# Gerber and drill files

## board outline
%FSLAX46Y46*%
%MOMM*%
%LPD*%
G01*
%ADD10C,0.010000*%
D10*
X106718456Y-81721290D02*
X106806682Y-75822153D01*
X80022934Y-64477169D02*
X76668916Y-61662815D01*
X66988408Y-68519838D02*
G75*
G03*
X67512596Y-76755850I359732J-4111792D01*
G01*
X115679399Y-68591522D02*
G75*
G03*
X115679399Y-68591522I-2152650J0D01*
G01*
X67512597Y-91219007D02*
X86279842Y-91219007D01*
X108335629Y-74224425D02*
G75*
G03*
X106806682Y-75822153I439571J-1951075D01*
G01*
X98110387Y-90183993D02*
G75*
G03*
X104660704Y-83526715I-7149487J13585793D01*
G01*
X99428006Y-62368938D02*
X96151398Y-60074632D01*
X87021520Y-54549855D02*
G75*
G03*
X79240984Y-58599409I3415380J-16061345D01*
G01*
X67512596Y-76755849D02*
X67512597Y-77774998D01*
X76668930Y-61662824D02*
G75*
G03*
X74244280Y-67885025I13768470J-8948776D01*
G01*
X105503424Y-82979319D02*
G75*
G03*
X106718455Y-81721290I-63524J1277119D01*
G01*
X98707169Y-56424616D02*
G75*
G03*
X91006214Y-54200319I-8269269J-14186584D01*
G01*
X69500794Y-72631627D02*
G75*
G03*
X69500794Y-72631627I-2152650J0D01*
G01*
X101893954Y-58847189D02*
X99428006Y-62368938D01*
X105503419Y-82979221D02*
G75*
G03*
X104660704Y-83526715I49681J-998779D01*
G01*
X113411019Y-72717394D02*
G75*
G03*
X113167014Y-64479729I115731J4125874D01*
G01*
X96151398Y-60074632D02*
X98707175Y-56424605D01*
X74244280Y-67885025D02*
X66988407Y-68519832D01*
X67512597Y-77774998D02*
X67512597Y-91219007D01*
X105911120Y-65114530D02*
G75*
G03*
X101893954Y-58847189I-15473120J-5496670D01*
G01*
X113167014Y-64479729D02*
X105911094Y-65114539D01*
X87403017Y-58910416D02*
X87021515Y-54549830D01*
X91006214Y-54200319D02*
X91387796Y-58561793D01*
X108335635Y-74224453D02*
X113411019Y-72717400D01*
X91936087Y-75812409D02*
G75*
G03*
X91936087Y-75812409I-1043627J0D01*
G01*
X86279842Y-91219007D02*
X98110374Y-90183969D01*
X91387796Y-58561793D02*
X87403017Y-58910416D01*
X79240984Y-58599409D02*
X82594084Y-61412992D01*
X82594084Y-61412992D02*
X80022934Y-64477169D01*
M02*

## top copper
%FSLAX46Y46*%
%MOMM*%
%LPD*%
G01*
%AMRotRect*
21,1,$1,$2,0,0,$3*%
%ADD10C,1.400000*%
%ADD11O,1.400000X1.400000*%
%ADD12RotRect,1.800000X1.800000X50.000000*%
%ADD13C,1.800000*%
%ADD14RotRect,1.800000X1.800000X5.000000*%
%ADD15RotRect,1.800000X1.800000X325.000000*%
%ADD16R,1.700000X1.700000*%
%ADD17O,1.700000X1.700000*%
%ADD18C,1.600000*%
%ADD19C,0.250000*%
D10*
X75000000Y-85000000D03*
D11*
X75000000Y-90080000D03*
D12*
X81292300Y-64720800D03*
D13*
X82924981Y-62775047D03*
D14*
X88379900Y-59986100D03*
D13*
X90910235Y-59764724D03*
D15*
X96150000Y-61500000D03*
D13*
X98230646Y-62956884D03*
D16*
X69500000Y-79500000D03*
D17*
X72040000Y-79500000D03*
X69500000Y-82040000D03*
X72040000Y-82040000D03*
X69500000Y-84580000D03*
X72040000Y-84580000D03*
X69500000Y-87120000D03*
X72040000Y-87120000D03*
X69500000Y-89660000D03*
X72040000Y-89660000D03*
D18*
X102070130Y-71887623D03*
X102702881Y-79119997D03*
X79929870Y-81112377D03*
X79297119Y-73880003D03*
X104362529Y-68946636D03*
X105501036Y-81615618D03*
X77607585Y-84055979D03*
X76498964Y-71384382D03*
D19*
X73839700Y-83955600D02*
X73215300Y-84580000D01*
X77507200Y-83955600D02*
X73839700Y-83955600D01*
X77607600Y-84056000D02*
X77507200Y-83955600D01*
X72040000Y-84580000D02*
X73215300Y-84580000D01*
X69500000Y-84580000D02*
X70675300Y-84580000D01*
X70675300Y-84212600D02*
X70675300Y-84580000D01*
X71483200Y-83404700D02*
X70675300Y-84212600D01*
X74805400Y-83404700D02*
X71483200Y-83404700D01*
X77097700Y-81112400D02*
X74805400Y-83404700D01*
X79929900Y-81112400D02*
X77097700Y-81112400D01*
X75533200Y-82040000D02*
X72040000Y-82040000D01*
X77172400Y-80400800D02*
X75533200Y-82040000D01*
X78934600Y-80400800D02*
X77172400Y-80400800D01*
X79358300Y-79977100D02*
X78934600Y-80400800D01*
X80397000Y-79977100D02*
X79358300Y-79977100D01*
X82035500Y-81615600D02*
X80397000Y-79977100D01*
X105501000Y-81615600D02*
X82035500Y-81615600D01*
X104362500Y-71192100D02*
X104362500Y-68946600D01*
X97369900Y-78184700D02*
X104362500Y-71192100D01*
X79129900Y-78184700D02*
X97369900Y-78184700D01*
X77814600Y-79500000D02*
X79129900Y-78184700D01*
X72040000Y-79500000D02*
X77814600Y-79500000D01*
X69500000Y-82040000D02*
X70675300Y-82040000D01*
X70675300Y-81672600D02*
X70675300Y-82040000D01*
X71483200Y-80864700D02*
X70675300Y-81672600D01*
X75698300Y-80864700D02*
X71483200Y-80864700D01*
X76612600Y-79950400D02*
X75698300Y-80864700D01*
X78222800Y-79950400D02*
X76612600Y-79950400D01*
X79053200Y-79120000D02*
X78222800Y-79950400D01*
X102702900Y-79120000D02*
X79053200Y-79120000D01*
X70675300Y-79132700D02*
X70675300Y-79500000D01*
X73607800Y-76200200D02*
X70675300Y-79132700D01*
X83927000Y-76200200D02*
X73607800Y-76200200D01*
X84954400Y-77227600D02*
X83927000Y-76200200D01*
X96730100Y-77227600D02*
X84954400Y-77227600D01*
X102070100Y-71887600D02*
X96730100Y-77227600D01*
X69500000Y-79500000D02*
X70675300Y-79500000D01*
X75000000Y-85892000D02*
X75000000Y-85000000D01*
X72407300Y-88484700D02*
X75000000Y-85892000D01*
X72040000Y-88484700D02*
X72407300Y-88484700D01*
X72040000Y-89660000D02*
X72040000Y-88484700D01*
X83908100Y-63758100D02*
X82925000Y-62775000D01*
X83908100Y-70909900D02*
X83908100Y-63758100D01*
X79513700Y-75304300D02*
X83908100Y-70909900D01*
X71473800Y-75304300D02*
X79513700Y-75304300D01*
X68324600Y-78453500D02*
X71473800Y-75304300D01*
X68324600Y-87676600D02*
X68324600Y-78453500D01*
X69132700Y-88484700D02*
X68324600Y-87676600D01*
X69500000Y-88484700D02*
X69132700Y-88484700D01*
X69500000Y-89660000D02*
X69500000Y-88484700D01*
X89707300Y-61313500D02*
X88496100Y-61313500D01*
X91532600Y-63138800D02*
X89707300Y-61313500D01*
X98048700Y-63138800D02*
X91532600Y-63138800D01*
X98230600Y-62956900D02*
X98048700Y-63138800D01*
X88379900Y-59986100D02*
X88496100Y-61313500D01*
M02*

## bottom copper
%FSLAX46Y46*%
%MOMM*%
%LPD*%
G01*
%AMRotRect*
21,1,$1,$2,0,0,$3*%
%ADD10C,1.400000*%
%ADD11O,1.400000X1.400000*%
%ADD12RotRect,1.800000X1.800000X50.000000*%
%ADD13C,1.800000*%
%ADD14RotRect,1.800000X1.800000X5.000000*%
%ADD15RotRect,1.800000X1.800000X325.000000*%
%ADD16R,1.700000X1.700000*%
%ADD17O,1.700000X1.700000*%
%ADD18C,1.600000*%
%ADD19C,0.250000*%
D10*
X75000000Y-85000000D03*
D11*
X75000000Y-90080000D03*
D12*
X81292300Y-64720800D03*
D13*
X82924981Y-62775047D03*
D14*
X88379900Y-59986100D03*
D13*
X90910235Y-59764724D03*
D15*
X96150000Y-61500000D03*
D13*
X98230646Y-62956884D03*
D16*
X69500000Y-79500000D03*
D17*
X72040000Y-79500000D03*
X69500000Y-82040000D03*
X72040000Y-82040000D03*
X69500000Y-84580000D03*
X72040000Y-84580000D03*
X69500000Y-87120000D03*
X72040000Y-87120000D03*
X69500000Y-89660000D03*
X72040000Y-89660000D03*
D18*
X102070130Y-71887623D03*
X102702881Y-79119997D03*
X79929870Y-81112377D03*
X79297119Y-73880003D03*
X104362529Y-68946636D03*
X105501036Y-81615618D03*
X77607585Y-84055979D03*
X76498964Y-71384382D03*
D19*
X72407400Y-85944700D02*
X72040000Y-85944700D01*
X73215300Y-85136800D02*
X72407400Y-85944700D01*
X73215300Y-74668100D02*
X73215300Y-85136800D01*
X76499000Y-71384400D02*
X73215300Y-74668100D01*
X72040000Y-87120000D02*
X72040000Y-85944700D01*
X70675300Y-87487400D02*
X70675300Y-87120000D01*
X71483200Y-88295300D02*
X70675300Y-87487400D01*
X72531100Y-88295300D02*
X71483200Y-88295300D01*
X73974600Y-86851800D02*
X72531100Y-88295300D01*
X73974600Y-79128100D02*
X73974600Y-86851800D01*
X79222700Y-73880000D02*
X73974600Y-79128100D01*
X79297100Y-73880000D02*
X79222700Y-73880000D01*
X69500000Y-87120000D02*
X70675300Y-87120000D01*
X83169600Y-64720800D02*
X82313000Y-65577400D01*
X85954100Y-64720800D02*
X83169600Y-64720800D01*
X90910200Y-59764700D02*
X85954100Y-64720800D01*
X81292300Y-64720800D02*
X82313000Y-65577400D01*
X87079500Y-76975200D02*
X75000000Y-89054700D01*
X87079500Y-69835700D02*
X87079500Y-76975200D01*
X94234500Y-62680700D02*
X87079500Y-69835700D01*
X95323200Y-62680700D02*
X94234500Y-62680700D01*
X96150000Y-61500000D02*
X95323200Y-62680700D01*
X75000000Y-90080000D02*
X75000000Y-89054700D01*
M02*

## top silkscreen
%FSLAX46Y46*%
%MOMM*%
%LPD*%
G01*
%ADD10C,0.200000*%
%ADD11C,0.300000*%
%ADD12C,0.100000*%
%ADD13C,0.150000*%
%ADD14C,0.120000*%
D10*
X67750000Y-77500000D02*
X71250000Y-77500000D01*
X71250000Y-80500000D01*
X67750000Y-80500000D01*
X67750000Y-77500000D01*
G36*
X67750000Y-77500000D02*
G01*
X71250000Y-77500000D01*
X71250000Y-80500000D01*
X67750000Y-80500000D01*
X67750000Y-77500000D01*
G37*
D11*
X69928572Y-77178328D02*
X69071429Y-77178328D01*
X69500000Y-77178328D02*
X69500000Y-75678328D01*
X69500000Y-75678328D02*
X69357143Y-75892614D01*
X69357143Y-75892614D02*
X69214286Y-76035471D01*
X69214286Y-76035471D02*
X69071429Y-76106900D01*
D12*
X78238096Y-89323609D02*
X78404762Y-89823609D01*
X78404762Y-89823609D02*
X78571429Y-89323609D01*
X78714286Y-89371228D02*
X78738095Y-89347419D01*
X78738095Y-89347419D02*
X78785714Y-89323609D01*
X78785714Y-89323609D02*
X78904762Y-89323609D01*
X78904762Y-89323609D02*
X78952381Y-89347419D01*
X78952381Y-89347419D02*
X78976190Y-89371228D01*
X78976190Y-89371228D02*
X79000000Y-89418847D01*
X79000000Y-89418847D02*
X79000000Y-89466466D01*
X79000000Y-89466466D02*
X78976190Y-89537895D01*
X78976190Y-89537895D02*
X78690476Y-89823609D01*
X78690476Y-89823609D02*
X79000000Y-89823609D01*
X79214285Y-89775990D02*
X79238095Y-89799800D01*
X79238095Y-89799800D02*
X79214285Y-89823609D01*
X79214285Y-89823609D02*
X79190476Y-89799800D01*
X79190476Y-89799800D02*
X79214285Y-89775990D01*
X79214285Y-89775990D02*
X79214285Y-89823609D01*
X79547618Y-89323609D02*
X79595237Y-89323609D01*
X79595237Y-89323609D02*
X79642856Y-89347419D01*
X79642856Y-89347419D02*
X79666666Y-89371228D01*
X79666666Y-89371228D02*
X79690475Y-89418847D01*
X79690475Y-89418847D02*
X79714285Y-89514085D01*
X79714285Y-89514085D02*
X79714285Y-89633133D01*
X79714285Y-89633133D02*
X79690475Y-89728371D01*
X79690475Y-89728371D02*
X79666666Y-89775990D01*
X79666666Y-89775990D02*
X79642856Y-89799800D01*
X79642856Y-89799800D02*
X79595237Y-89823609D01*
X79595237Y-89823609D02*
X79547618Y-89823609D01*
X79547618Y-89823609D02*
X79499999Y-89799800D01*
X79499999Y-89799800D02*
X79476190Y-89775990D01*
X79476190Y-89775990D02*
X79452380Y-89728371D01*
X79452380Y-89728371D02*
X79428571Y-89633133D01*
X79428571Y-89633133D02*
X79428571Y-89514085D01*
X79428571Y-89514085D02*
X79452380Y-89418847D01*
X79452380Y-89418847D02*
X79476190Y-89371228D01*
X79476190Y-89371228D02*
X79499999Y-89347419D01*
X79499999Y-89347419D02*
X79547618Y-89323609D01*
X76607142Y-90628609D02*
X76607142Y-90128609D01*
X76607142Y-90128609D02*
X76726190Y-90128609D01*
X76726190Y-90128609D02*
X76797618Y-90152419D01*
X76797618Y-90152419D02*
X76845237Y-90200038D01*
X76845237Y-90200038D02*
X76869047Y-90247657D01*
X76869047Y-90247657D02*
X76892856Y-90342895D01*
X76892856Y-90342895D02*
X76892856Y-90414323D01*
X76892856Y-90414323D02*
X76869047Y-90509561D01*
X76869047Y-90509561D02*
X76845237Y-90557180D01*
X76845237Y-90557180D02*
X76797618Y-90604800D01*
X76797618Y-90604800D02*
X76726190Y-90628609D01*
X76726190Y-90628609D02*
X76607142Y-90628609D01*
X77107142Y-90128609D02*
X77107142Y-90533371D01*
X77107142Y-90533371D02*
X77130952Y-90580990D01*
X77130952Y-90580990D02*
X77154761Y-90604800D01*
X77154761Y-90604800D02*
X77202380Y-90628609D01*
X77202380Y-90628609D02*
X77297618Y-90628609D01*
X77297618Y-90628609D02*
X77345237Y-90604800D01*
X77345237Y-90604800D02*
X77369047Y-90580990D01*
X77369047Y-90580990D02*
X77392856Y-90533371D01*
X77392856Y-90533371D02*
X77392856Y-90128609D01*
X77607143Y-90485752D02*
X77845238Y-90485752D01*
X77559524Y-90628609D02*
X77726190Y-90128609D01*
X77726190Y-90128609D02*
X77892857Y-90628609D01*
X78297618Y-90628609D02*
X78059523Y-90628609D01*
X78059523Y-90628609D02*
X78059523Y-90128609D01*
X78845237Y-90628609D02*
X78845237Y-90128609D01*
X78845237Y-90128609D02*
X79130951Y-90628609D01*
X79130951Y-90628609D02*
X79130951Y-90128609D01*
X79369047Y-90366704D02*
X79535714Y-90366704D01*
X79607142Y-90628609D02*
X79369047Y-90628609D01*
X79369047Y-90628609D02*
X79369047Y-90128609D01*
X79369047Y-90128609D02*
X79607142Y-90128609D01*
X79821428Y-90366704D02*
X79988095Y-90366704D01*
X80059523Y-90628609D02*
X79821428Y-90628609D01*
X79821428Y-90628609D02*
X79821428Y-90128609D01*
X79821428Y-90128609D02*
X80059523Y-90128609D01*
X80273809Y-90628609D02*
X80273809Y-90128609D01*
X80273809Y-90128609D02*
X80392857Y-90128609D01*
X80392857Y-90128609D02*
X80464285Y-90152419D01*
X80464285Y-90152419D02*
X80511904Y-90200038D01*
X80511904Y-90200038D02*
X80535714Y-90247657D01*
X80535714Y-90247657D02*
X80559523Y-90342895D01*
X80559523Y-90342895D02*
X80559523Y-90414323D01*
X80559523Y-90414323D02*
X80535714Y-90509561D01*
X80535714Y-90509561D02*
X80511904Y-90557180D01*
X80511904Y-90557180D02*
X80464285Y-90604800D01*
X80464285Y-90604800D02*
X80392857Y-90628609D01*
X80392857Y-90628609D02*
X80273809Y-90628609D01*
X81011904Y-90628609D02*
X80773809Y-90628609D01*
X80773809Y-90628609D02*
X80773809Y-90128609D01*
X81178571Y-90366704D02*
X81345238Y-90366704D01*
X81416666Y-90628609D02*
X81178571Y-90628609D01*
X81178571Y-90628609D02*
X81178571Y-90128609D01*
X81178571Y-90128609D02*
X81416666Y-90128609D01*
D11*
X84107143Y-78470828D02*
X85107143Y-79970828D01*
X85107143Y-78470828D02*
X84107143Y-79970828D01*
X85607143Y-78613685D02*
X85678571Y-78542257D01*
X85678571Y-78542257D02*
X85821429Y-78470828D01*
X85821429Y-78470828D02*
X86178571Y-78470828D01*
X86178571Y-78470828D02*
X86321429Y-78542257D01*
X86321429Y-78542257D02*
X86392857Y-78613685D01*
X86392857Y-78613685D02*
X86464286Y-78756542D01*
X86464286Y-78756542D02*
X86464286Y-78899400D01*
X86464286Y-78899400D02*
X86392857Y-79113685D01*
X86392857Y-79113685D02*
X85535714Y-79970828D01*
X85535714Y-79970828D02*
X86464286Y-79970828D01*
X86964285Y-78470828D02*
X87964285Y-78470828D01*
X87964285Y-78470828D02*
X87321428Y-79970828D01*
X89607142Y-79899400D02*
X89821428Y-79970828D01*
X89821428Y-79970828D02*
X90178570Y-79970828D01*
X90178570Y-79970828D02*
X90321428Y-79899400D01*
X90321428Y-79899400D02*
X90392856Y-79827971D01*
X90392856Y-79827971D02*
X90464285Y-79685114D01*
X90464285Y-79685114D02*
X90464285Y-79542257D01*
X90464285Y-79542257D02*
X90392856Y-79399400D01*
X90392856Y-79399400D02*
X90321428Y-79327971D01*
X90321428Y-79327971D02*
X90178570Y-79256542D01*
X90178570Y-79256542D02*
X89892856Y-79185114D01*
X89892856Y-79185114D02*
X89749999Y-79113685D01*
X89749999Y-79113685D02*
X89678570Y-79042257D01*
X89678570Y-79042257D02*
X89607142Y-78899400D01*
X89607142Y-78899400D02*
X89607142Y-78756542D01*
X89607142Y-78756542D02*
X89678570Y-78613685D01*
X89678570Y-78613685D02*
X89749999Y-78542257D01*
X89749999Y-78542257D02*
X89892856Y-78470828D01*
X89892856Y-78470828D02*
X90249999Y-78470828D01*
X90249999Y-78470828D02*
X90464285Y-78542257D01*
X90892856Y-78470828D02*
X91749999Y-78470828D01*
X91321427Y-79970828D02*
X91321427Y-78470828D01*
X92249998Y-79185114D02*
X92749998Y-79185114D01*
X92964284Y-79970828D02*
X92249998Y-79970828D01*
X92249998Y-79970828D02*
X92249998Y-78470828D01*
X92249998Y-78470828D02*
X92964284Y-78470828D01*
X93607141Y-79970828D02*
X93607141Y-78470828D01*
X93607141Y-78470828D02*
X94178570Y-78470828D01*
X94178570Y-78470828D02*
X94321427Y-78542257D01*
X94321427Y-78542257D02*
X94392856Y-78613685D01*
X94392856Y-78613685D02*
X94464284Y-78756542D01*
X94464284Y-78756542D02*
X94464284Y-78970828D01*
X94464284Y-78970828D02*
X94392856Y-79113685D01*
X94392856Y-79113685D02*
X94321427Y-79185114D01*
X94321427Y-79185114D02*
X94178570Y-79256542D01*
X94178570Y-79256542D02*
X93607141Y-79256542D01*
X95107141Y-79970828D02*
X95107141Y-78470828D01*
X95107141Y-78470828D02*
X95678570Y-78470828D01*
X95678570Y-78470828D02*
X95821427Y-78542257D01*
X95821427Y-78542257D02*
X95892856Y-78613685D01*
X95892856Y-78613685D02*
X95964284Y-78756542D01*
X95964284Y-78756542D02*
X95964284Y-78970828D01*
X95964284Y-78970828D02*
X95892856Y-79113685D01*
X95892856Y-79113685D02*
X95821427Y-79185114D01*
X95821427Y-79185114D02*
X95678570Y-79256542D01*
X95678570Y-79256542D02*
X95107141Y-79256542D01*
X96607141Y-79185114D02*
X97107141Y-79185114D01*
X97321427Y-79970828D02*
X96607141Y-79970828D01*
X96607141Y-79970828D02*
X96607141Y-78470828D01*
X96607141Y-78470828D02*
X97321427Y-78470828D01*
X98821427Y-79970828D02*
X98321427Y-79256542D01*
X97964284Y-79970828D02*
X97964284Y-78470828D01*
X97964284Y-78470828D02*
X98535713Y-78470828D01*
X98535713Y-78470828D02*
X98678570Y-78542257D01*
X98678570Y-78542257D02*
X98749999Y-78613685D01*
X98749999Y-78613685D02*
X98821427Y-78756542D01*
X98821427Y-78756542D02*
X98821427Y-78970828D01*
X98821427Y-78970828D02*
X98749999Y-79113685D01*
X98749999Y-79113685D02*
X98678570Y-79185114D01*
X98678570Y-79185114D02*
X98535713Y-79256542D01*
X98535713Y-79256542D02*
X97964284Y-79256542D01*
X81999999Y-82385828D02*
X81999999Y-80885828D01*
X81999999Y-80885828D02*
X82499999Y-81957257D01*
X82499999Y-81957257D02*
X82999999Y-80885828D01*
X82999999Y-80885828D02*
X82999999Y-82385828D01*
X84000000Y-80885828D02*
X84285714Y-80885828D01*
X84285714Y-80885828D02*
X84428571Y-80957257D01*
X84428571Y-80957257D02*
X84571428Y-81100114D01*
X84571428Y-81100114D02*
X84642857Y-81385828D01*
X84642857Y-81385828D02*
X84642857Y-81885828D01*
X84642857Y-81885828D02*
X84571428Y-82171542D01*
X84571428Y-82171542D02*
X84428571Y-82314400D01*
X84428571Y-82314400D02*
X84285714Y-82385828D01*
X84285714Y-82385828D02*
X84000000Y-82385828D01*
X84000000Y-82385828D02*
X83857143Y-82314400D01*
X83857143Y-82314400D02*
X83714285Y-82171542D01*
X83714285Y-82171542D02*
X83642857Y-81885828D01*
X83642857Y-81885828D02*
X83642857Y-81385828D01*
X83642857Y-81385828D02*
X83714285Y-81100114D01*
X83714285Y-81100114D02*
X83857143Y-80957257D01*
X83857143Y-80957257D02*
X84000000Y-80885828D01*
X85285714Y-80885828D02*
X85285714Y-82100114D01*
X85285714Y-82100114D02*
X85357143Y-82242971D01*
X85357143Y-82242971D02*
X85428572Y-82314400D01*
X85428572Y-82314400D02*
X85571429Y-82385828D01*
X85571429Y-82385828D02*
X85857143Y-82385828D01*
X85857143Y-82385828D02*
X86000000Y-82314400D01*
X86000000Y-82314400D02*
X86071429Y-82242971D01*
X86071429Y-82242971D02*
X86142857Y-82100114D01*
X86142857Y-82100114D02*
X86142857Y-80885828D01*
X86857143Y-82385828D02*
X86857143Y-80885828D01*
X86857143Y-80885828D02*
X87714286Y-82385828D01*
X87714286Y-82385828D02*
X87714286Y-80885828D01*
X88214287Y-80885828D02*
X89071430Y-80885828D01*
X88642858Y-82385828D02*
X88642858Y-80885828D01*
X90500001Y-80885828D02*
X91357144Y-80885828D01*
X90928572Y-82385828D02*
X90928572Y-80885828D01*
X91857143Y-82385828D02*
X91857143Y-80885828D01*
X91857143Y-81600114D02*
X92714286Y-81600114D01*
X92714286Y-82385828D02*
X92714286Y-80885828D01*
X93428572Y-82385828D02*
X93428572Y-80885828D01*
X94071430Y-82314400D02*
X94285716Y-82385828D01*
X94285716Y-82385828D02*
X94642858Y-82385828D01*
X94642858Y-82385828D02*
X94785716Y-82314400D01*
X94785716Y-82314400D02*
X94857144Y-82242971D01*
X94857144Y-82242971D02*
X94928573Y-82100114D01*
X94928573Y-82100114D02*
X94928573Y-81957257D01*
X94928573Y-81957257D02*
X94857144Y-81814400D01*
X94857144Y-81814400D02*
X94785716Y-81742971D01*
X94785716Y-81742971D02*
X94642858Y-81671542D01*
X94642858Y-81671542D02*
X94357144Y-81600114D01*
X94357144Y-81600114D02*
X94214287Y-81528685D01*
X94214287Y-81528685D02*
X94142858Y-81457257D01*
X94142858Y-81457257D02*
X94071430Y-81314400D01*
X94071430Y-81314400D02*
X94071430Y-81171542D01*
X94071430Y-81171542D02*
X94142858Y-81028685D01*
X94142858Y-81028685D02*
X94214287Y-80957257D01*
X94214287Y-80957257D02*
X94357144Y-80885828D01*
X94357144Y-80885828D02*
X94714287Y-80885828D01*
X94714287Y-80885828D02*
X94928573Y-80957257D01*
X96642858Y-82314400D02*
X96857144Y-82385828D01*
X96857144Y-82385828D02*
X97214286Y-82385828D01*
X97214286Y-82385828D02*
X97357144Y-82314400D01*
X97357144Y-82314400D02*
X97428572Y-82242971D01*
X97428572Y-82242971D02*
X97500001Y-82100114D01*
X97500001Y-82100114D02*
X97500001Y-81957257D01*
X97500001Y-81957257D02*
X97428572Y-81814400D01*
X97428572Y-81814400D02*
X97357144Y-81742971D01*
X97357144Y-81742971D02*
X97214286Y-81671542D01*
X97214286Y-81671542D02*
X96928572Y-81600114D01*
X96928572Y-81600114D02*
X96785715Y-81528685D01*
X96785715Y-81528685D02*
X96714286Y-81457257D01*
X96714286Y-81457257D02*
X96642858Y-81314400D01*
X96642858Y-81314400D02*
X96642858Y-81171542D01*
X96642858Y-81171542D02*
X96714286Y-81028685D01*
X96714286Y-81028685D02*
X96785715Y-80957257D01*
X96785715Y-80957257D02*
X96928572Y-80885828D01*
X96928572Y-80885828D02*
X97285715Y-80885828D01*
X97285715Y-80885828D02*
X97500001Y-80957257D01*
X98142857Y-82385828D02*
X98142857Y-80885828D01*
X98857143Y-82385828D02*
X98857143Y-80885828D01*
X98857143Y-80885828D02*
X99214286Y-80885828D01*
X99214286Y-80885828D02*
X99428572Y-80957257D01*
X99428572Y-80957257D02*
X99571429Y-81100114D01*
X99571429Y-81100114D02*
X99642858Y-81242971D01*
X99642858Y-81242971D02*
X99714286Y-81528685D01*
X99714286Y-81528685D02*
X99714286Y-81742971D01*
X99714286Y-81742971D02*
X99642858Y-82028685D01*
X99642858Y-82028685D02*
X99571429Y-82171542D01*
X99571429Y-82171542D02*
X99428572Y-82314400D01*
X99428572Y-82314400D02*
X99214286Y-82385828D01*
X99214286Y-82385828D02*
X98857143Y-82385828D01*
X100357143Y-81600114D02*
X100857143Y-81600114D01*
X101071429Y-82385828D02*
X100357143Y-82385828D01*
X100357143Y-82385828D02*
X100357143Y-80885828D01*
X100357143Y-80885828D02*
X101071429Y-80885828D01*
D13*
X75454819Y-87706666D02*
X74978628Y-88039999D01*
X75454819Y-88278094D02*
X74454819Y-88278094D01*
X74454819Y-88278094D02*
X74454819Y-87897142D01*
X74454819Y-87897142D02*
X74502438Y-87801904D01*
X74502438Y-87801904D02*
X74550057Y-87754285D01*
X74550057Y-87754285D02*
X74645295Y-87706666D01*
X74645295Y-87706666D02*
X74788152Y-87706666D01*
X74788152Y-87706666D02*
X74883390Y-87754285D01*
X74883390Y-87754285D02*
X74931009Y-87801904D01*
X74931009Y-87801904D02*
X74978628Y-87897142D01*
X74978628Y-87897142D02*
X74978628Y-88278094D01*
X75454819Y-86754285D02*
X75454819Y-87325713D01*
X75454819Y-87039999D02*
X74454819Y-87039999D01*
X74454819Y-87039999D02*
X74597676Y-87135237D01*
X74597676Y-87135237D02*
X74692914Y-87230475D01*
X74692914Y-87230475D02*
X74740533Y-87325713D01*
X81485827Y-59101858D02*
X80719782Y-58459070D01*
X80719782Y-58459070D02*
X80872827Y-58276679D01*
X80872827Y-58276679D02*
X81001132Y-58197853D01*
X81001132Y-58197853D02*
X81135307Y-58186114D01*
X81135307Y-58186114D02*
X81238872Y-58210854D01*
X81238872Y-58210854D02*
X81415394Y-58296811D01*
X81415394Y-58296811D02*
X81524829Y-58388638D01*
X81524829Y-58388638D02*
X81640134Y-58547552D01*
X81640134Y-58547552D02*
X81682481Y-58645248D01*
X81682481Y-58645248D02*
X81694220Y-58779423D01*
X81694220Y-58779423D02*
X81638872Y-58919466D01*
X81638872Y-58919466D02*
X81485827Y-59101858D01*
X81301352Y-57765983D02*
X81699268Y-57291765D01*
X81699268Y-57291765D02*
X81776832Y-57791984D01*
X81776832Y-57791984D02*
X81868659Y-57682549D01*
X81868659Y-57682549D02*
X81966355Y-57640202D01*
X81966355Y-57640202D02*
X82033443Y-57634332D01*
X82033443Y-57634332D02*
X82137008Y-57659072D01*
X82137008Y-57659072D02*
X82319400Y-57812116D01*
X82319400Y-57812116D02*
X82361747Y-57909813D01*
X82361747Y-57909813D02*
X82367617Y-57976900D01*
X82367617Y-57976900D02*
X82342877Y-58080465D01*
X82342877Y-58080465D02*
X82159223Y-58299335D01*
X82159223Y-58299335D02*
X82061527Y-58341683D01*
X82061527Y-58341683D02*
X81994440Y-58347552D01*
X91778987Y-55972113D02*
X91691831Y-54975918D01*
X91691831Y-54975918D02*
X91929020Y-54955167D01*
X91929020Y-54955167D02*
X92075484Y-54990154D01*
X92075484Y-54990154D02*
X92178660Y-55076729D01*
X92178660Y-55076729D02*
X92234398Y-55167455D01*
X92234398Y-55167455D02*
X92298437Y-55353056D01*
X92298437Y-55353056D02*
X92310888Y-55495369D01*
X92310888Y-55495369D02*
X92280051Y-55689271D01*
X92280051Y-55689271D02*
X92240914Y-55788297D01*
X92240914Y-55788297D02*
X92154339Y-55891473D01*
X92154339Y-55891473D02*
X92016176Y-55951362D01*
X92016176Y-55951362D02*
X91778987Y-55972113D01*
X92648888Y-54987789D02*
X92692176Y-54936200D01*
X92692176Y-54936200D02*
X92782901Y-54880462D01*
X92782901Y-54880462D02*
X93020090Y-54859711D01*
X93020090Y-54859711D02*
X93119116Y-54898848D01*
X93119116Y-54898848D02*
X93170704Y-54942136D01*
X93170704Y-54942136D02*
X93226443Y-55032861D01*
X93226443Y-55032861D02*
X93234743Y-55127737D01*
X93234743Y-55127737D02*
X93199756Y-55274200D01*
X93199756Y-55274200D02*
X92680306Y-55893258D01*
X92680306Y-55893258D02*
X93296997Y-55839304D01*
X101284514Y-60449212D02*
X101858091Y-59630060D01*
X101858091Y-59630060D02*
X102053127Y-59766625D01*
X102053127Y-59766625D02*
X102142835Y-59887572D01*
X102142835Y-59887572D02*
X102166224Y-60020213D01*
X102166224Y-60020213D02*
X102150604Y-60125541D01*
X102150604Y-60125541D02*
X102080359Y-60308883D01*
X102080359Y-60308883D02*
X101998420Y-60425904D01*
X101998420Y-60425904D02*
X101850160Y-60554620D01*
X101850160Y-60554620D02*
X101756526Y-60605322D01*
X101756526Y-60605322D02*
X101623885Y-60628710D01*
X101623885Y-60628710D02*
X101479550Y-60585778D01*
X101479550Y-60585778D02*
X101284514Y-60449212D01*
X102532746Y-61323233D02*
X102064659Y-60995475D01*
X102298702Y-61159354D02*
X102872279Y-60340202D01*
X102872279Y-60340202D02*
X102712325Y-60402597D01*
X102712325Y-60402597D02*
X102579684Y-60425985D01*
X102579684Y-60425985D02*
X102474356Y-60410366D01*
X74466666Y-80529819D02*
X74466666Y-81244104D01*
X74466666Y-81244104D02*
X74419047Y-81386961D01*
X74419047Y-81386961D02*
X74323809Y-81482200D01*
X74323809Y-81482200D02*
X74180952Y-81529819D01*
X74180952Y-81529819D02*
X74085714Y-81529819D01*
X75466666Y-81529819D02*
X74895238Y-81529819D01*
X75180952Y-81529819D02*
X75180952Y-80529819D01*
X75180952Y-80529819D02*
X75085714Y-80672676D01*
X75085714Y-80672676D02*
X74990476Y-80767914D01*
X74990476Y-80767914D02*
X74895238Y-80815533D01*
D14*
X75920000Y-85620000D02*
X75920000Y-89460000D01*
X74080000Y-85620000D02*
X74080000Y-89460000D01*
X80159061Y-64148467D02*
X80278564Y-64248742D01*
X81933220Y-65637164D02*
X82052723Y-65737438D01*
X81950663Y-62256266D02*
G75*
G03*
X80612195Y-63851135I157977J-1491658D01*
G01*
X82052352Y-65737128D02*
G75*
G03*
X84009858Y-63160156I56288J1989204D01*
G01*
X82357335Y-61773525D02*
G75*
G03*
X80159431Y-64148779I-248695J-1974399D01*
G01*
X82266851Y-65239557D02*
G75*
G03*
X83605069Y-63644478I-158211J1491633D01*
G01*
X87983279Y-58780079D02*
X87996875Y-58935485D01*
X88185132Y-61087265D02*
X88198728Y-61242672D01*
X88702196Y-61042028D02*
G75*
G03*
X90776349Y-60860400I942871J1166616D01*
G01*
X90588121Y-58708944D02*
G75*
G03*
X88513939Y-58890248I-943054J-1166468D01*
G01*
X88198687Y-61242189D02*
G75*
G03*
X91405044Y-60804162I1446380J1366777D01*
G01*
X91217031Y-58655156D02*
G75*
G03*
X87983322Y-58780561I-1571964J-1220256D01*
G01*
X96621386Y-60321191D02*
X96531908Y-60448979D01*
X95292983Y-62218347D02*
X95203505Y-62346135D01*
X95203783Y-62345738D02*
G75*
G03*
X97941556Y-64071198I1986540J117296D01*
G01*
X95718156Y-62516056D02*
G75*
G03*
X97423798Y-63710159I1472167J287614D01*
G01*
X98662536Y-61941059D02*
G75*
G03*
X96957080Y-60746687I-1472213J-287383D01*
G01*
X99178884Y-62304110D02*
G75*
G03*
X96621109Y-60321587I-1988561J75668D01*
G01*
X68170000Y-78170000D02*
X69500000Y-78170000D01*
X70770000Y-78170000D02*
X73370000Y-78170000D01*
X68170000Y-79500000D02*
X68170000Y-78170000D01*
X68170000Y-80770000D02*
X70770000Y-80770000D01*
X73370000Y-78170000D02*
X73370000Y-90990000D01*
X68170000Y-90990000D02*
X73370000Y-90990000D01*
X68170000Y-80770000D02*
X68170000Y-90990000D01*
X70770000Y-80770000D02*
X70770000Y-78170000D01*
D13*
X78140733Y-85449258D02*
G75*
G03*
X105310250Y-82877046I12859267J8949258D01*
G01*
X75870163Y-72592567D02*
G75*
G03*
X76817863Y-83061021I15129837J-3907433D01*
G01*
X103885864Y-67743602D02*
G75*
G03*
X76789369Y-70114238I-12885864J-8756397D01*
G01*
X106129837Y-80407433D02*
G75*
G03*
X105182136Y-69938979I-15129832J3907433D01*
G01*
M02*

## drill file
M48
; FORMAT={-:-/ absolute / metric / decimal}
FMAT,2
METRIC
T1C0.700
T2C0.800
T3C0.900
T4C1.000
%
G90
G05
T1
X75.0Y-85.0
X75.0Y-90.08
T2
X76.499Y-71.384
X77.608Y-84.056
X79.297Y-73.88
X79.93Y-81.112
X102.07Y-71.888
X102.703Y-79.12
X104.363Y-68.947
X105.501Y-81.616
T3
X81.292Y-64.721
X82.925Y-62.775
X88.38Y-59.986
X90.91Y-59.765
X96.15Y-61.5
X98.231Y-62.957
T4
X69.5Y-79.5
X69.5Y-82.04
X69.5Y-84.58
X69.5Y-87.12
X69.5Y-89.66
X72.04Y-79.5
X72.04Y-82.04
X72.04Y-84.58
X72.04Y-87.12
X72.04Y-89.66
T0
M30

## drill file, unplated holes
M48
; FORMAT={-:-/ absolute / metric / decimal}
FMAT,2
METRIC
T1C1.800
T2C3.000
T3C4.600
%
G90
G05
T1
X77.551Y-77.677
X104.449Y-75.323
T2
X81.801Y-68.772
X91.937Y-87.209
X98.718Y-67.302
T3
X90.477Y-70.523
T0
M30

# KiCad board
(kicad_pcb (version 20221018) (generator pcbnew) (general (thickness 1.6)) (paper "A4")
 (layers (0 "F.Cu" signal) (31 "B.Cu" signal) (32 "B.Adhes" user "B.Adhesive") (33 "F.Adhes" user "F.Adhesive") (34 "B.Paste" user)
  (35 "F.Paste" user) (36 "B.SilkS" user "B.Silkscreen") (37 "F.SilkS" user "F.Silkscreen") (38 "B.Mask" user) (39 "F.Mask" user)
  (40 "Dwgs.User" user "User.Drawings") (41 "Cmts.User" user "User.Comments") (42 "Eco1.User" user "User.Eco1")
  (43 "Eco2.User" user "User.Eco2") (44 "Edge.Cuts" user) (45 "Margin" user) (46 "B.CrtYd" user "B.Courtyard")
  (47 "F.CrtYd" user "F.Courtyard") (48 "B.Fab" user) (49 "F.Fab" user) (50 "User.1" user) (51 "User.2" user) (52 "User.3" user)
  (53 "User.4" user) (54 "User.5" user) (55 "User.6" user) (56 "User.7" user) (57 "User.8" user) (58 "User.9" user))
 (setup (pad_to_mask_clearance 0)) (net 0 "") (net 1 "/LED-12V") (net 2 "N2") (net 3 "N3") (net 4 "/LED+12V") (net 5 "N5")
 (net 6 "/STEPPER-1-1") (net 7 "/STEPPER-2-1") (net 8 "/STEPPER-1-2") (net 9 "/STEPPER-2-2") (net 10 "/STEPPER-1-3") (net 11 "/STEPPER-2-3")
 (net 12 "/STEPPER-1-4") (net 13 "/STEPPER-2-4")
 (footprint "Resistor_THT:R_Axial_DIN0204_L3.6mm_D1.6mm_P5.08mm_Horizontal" (layer "F.Cu") (at 75 85 -90)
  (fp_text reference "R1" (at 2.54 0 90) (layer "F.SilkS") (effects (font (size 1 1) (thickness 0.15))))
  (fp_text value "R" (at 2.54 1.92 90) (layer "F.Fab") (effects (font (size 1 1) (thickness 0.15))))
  (fp_line (start 0.62 -0.92) (end 4.46 -0.92) (stroke (width 0.12) (type solid)) (layer "F.SilkS"))
  (fp_line (start 0.62 0.92) (end 4.46 0.92) (stroke (width 0.12) (type solid)) (layer "F.SilkS"))
  (pad "1" thru_hole circle (at 0 0 270) (size 1.4 1.4) (drill 0.7) (layers "*.Cu" "*.Mask") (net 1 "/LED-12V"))
  (pad "2" thru_hole oval (at 5.08 0 270) (size 1.4 1.4) (drill 0.7) (layers "*.Cu" "*.Mask") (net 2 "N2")))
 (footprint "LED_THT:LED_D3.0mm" (layer "F.Cu") (at 81.2923 64.7208 50)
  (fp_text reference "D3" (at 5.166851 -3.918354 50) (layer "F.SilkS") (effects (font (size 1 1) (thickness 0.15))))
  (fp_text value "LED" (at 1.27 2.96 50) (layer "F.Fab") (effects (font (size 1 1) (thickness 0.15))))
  (fp_line (start -0.29 -1.236) (end -0.29 -1.08) (stroke (width 0.12) (type solid)) (layer "F.SilkS"))
  (fp_line (start -0.29 1.08) (end -0.29 1.236) (stroke (width 0.12) (type solid)) (layer "F.SilkS"))
  (fp_arc (start -0.29 -1.235516) (mid 1.366488 -1.987659) (end 2.942335 -1.078608) (stroke (width 0.12) (type solid)) (layer "F.SilkS"))
  (fp_arc (start 0.229039 -1.08) (mid 1.270117 -1.5) (end 2.31113 -1.079837) (stroke (width 0.12) (type solid)) (layer "F.SilkS"))
  (fp_arc (start 2.31113 1.079837) (mid 1.270117 1.5) (end 0.229039 1.08) (stroke (width 0.12) (type solid)) (layer "F.SilkS"))
  (fp_arc (start 2.942335 1.078608) (mid 1.366487 1.987659) (end -0.29 1.235516) (stroke (width 0.12) (type solid)) (layer "F.SilkS"))
  (pad "1" thru_hole rect (at 0 0 50) (size 1.8 1.8) (drill 0.9) (layers "*.Cu" "*.Mask") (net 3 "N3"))
  (pad "2" thru_hole circle (at 2.54 0 50) (size 1.8 1.8) (drill 0.9) (layers "*.Cu" "*.Mask") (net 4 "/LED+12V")))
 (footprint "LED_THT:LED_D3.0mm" (layer "F.Cu") (at 88.3799 59.9861 5)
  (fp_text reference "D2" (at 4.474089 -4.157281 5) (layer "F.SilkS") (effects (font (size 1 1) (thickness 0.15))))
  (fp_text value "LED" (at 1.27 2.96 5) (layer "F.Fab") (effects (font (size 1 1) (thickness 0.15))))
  (fp_line (start -0.29 -1.236) (end -0.29 -1.08) (stroke (width 0.12) (type solid)) (layer "F.SilkS"))
  (fp_line (start -0.29 1.08) (end -0.29 1.236) (stroke (width 0.12) (type solid)) (layer "F.SilkS"))
  (fp_arc (start -0.29 -1.235516) (mid 1.366488 -1.987659) (end 2.942335 -1.078608) (stroke (width 0.12) (type solid)) (layer "F.SilkS"))
  (fp_arc (start 0.229039 -1.08) (mid 1.270118 -1.5) (end 2.31113 -1.079837) (stroke (width 0.12) (type solid)) (layer "F.SilkS"))
  (fp_arc (start 2.31113 1.079837) (mid 1.270118 1.5) (end 0.229039 1.08) (stroke (width 0.12) (type solid)) (layer "F.SilkS"))
  (fp_arc (start 2.942335 1.078608) (mid 1.366488 1.987659) (end -0.29 1.235516) (stroke (width 0.12) (type solid)) (layer "F.SilkS"))
  (pad "1" thru_hole rect (at 0 0 5) (size 1.8 1.8) (drill 0.9) (layers "*.Cu" "*.Mask") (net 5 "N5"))
  (pad "2" thru_hole circle (at 2.54 0 5) (size 1.8 1.8) (drill 0.9) (layers "*.Cu" "*.Mask") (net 3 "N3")))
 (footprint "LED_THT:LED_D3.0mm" (layer "F.Cu") (at 96.15 61.5 -35)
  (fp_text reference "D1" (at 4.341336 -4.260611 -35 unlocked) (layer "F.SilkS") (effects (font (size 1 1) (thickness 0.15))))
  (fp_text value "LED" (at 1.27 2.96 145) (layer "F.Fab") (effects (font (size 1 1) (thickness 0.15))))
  (fp_line (start -0.29 -1.236) (end -0.29 -1.08) (stroke (width 0.12) (type solid)) (layer "F.SilkS"))
  (fp_line (start -0.29 1.08) (end -0.29 1.236) (stroke (width 0.12) (type solid)) (layer "F.SilkS"))
  (fp_arc (start -0.29 -1.235516) (mid 1.366487 -1.987659) (end 2.942335 -1.078608) (stroke (width 0.12) (type solid)) (layer "F.SilkS"))
  (fp_arc (start 0.229039 -1.08) (mid 1.270118 -1.5) (end 2.31113 -1.079837) (stroke (width 0.12) (type solid)) (layer "F.SilkS"))
  (fp_arc (start 2.31113 1.079837) (mid 1.270117 1.5) (end 0.229039 1.08) (stroke (width 0.12) (type solid)) (layer "F.SilkS"))
  (fp_arc (start 2.942335 1.078608) (mid 1.366487 1.987659) (end -0.29 1.235516) (stroke (width 0.12) (type solid)) (layer "F.SilkS"))
  (pad "1" thru_hole rect (at 0 0 325) (size 1.8 1.8) (drill 0.9) (layers "*.Cu" "*.Mask") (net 2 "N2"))
  (pad "2" thru_hole circle (at 2.54 0 325) (size 1.8 1.8) (drill 0.9) (layers "*.Cu" "*.Mask") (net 5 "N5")))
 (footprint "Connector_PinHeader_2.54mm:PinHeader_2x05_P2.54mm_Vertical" (layer "F.Cu") (at 69.5 79.5)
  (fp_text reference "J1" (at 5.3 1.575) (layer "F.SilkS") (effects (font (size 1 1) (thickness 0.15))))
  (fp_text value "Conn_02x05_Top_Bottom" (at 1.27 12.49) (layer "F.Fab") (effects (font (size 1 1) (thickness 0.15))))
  (fp_line (start -1.33 -1.33) (end 0 -1.33) (stroke (width 0.12) (type solid)) (layer "F.SilkS"))
  (fp_line (start -1.33 0) (end -1.33 -1.33) (stroke (width 0.12) (type solid)) (layer "F.SilkS"))
  (fp_line (start -1.33 1.27) (end -1.33 11.49) (stroke (width 0.12) (type solid)) (layer "F.SilkS"))
  (fp_line (start -1.33 1.27) (end 1.27 1.27) (stroke (width 0.12) (type solid)) (layer "F.SilkS"))
  (fp_line (start -1.33 11.49) (end 3.87 11.49) (stroke (width 0.12) (type solid)) (layer "F.SilkS"))
  (fp_line (start 1.27 -1.33) (end 3.87 -1.33) (stroke (width 0.12) (type solid)) (layer "F.SilkS"))
  (fp_line (start 1.27 1.27) (end 1.27 -1.33) (stroke (width 0.12) (type solid)) (layer "F.SilkS"))
  (fp_line (start 3.87 -1.33) (end 3.87 11.49) (stroke (width 0.12) (type solid)) (layer "F.SilkS"))
  (pad "1" thru_hole rect (at 0 0) (size 1.7 1.7) (drill 1) (layers "*.Cu" "*.Mask") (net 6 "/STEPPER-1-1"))
  (pad "2" thru_hole oval (at 2.54 0) (size 1.7 1.7) (drill 1) (layers "*.Cu" "*.Mask") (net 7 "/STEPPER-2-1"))
  (pad "3" thru_hole oval (at 0 2.54) (size 1.7 1.7) (drill 1) (layers "*.Cu" "*.Mask") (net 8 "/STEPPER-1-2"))
  (pad "4" thru_hole oval (at 2.54 2.54) (size 1.7 1.7) (drill 1) (layers "*.Cu" "*.Mask") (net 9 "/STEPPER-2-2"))
  (pad "5" thru_hole oval (at 0 5.08) (size 1.7 1.7) (drill 1) (layers "*.Cu" "*.Mask") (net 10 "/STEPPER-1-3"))
  (pad "6" thru_hole oval (at 2.54 5.08) (size 1.7 1.7) (drill 1) (layers "*.Cu" "*.Mask") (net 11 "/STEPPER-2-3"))
  (pad "7" thru_hole oval (at 0 7.62) (size 1.7 1.7) (drill 1) (layers "*.Cu" "*.Mask") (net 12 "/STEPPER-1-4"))
  (pad "8" thru_hole oval (at 2.54 7.62) (size 1.7 1.7) (drill 1) (layers "*.Cu" "*.Mask") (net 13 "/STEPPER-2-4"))
  (pad "9" thru_hole oval (at 0 10.16) (size 1.7 1.7) (drill 1) (layers "*.Cu" "*.Mask") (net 4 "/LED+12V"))
  (pad "10" thru_hole oval (at 2.54 10.16) (size 1.7 1.7) (drill 1) (layers "*.Cu" "*.Mask") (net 1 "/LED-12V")))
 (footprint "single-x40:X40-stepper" (layer "B.Cu") (at 91 76.5 -175)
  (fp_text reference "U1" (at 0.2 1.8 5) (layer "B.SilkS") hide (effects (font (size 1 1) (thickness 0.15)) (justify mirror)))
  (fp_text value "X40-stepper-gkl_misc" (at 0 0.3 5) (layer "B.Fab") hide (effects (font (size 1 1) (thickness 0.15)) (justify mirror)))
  (fp_arc (start -14.7 5.3) (mid -15.626189 0.047138) (end -14.731708 -5.211216) (stroke (width 0.15) (type solid)) (layer "F.SilkS"))
  (fp_arc (start -13.7 -7.6) (mid -0.111624 -15.666446) (end 13.590314 -7.794445) (stroke (width 0.15) (type solid)) (layer "F.SilkS"))
  (fp_arc (start 13.6 7.6) (mid 0 15.579474) (end -13.6 7.6) (stroke (width 0.15) (type solid)) (layer "F.SilkS"))
  (fp_arc (start 14.7 -5.3) (mid 15.626189 -0.047138) (end 14.731708 5.211216) (stroke (width 0.15) (type solid)) (layer "F.SilkS"))
  (pad "" np_thru_hole circle (at -13.5 0 185) (size 1.8 1.8) (drill 1.8) (layers "*.Cu" "*.Mask"))
  (pad "" np_thru_hole circle (at -8.49 8.49 185) (size 3 3) (drill 3) (layers "*.Cu" "*.Mask"))
  (pad "" np_thru_hole circle (at 0 -10.75 185) (size 3 3) (drill 3) (layers "*.Cu" "*.Mask"))
  (pad "" np_thru_hole circle (at 0 6 185) (size 4.6 4.6) (drill 4.6) (layers "*.Cu" "*.Mask"))
  (pad "" np_thru_hole circle (at 8.49 8.5 185) (size 3 3) (drill 3) (layers "*.Cu" "*.Mask"))
  (pad "" np_thru_hole circle (at 13.5 0 185) (size 1.8 1.8) (drill 1.8) (layers "*.Cu" "*.Mask"))
  (pad "1" thru_hole circle (at -11.43 3.63 185) (size 1.6 1.6) (drill 0.8) (layers "*.Cu" "*.Mask") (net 6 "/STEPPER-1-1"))
  (pad "2" thru_hole circle (at -11.43 -3.63 185) (size 1.6 1.6) (drill 0.8) (layers "*.Cu" "*.Mask") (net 8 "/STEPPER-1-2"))
  (pad "3" thru_hole circle (at 11.43 -3.63 185) (size 1.6 1.6) (drill 0.8) (layers "*.Cu" "*.Mask") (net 10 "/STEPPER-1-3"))
  (pad "4" thru_hole circle (at 11.43 3.63 185) (size 1.6 1.6) (drill 0.8) (layers "*.Cu" "*.Mask") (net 12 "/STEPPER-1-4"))
  (pad "5" thru_hole circle (at -13.97 6.36 185) (size 1.6 1.6) (drill 0.8) (layers "*.Cu" "*.Mask") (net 7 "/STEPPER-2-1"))
  (pad "6" thru_hole circle (at -14 -6.36 185) (size 1.6 1.6) (drill 0.8) (layers "*.Cu" "*.Mask") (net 9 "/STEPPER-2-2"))
  (pad "7" thru_hole circle (at 14 -6.36 185) (size 1.6 1.6) (drill 0.8) (layers "*.Cu" "*.Mask") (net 11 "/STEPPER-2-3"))
  (pad "8" thru_hole circle (at 14 6.36 185) (size 1.6 1.6) (drill 0.8) (layers "*.Cu" "*.Mask") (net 13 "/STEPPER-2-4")))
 (gr_rect (start 67.75 77.5) (end 71.25 80.5) (stroke (width 0.2) (type solid)) (fill solid) (layer "F.SilkS"))
 (gr_line (start 106.718456 81.72129) (end 106.806682 75.822153) (stroke (width 0.01) (type solid)) (layer "Edge.Cuts"))
 (gr_line (start 80.022934 64.477169) (end 76.668916 61.662815) (stroke (width 0.01) (type solid)) (layer "Edge.Cuts"))
 (gr_arc (start 67.512596 76.755851) (mid 63.228977 72.893795) (end 66.988407 68.519832) (stroke (width 0.01) (type solid))
  (layer "Edge.Cuts"))
 (gr_circle (center 113.526749 68.591522) (end 115.679399 68.591522) (stroke (width 0.01) (type solid)) (fill none) (layer "Edge.Cuts"))
 (gr_line (start 67.512597 91.219007) (end 86.279842 91.219007) (stroke (width 0.01) (type solid)) (layer "Edge.Cuts"))
 (gr_arc (start 106.806682 75.822153) (mid 107.330253 74.792764) (end 108.335635 74.224453) (stroke (width 0.01) (type solid))
  (layer "Edge.Cuts"))
 (gr_arc (start 104.660704 83.526715) (mid 101.904066 87.365541) (end 98.110374 90.183969) (stroke (width 0.01) (type solid))
  (layer "Edge.Cuts"))
 (gr_line (start 99.428006 62.368938) (end 96.151398 60.074632) (stroke (width 0.01) (type solid)) (layer "Edge.Cuts"))
 (gr_arc (start 79.240984 58.599409) (mid 82.855853 56.045494) (end 87.021515 54.54983) (stroke (width 0.01) (type solid))
  (layer "Edge.Cuts"))
 (gr_line (start 67.512596 76.755849) (end 67.512597 77.774998) (stroke (width 0.01) (type solid)) (layer "Edge.Cuts"))
 (gr_arc (start 74.24428 67.885025) (mid 75.136963 64.649366) (end 76.668916 61.662815) (stroke (width 0.01) (type solid))
  (layer "Edge.Cuts"))
 (gr_arc (start 106.718456 81.72129) (mid 106.359644 82.590491) (end 105.503421 82.979257) (stroke (width 0.01) (type solid))
  (layer "Edge.Cuts"))
 (gr_arc (start 91.006214 54.200319) (mid 94.994501 54.835344) (end 98.707175 56.424605) (stroke (width 0.01) (type solid))
  (layer "Edge.Cuts"))
 (gr_circle (center 67.348144 72.631627) (end 69.500794 72.631627) (stroke (width 0.01) (type solid)) (fill none) (layer "Edge.Cuts"))
 (gr_line (start 101.893954 58.847189) (end 99.428006 62.368938) (stroke (width 0.01) (type solid)) (layer "Edge.Cuts"))
 (gr_arc (start 104.660704 83.526715) (mid 105.008299 83.13944) (end 105.503421 82.979257) (stroke (width 0.01) (type solid))
  (layer "Edge.Cuts"))
 (gr_arc (start 113.167014 64.479729) (mid 117.65244 68.469317) (end 113.411019 72.7174) (stroke (width 0.01) (type solid))
  (layer "Edge.Cuts"))
 (gr_line (start 96.151398 60.074632) (end 98.707175 56.424605) (stroke (width 0.01) (type solid)) (layer "Edge.Cuts"))
 (gr_line (start 74.24428 67.885025) (end 66.988407 68.519832) (stroke (width 0.01) (type solid)) (layer "Edge.Cuts"))
 (gr_line (start 67.512597 77.774998) (end 67.512597 91.219007) (stroke (width 0.01) (type solid)) (layer "Edge.Cuts"))
 (gr_arc (start 101.893954 58.847189) (mid 104.262373 61.750214) (end 105.911094 65.114539) (stroke (width 0.01) (type solid))
  (layer "Edge.Cuts"))
 (gr_line (start 113.167014 64.479729) (end 105.911094 65.114539) (stroke (width 0.01) (type solid)) (layer "Edge.Cuts"))
 (gr_line (start 87.403017 58.910416) (end 87.021515 54.54983) (stroke (width 0.01) (type solid)) (layer "Edge.Cuts"))
 (gr_line (start 91.006214 54.200319) (end 91.387796 58.561793) (stroke (width 0.01) (type solid)) (layer "Edge.Cuts"))
 (gr_line (start 108.335635 74.224453) (end 113.411019 72.7174) (stroke (width 0.01) (type solid)) (layer "Edge.Cuts"))
 (gr_circle (center 90.89246 75.812409) (end 91.936087 75.812409) (stroke (width 0.01) (type solid)) (fill none) (layer "Edge.Cuts"))
 (gr_line (start 86.279842 91.219007) (end 98.110374 90.183969) (stroke (width 0.01) (type solid)) (layer "Edge.Cuts"))
 (gr_line (start 91.387796 58.561793) (end 87.403017 58.910416) (stroke (width 0.01) (type solid)) (layer "Edge.Cuts"))
 (gr_line (start 79.240984 58.599409) (end 82.594084 61.412992) (stroke (width 0.01) (type solid)) (layer "Edge.Cuts"))
 (gr_line (start 82.594084 61.412992) (end 80.022934 64.477169) (stroke (width 0.01) (type solid)) (layer "Edge.Cuts"))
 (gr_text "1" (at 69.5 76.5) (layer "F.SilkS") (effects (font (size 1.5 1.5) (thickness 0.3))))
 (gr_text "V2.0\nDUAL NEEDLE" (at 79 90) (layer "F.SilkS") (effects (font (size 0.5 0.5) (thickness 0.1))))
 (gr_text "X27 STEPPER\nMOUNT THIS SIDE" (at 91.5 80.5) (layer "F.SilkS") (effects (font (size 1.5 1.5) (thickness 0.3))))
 (segment (start 87.0795 76.9752) (end 75 89.0547) (width 0.25) (layer "B.Cu") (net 2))
 (segment (start 95.3232 62.6807) (end 94.2345 62.6807) (width 0.25) (layer "B.Cu") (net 2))
 (segment (start 96.15 61.5) (end 95.3232 62.6807) (width 0.25) (layer "B.Cu") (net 2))
 (segment (start 94.2345 62.6807) (end 87.0795 69.8357) (width 0.25) (layer "B.Cu") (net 2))
 (segment (start 87.0795 69.8357) (end 87.0795 76.9752) (width 0.25) (layer "B.Cu") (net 2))
 (segment (start 75 90.08) (end 75 89.0547) (width 0.25) (layer "B.Cu") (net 2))
 (segment (start 91.5326 63.1388) (end 89.7073 61.3135) (width 0.25) (layer "F.Cu") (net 5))
 (segment (start 98.2306 62.9569) (end 98.0487 63.1388) (width 0.25) (layer "F.Cu") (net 5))
 (segment (start 89.7073 61.3135) (end 88.4961 61.3135) (width 0.25) (layer "F.Cu") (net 5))
 (segment (start 88.3799 59.9861) (end 88.4961 61.3135) (width 0.25) (layer "F.Cu") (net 5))
 (segment (start 98.0487 63.1388) (end 91.5326 63.1388) (width 0.25) (layer "F.Cu") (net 5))
 (segment (start 90.9102 59.7647) (end 85.9541 64.7208) (width 0.25) (layer "B.Cu") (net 3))
 (segment (start 85.9541 64.7208) (end 83.1696 64.7208) (width 0.25) (layer "B.Cu") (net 3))
 (segment (start 83.1696 64.7208) (end 82.313 65.5774) (width 0.25) (layer "B.Cu") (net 3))
 (segment (start 81.2923 64.7208) (end 82.313 65.5774) (width 0.25) (layer "B.Cu") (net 3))
 (segment (start 83.9081 63.7581) (end 82.925 62.775) (width 0.25) (layer "F.Cu") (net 4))
 (segment (start 68.3246 78.4535) (end 71.4738 75.3043) (width 0.25) (layer "F.Cu") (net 4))
 (segment (start 69.1327 88.4847) (end 68.3246 87.6766) (width 0.25) (layer "F.Cu") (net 4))
 (segment (start 69.5 89.66) (end 69.5 88.4847) (width 0.25) (layer "F.Cu") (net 4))
 (segment (start 83.9081 70.9099) (end 83.9081 63.7581) (width 0.25) (layer "F.Cu") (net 4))
 (segment (start 68.3246 87.6766) (end 68.3246 78.4535) (width 0.25) (layer "F.Cu") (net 4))
 (segment (start 71.4738 75.3043) (end 79.5137 75.3043) (width 0.25) (layer "F.Cu") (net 4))
 (segment (start 79.5137 75.3043) (end 83.9081 70.9099) (width 0.25) (layer "F.Cu") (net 4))
 (segment (start 69.5 88.4847) (end 69.1327 88.4847) (width 0.25) (layer "F.Cu") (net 4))
 (segment (start 72.4073 88.4847) (end 75 85.892) (width 0.25) (layer "F.Cu") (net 1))
 (segment (start 75 85.892) (end 75 85) (width 0.25) (layer "F.Cu") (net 1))
 (segment (start 72.04 88.4847) (end 72.4073 88.4847) (width 0.25) (layer "F.Cu") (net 1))
 (segment (start 72.04 89.66) (end 72.04 88.4847) (width 0.25) (layer "F.Cu") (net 1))
 (segment (start 84.9544 77.2276) (end 83.927 76.2002) (width 0.25) (layer "F.Cu") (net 6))
 (segment (start 73.6078 76.2002) (end 70.6753 79.1327) (width 0.25) (layer "F.Cu") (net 6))
 (segment (start 102.0701 71.8876) (end 96.7301 77.2276) (width 0.25) (layer "F.Cu") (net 6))
 (segment (start 96.7301 77.2276) (end 84.9544 77.2276) (width 0.25) (layer "F.Cu") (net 6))
 (segment (start 69.5 79.5) (end 70.6753 79.5) (width 0.25) (layer "F.Cu") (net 6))
 (segment (start 70.6753 79.1327) (end 70.6753 79.5) (width 0.25) (layer "F.Cu") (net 6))
 (segment (start 83.927 76.2002) (end 73.6078 76.2002) (width 0.25) (layer "F.Cu") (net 6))
 (segment (start 78.2228 79.9504) (end 76.6126 79.9504) (width 0.25) (layer "F.Cu") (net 8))
 (segment (start 71.4832 80.8647) (end 70.6753 81.6726) (width 0.25) (layer "F.Cu") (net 8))
 (segment (start 75.6983 80.8647) (end 71.4832 80.8647) (width 0.25) (layer "F.Cu") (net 8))
 (segment (start 69.5 82.04) (end 70.6753 82.04) (width 0.25) (layer "F.Cu") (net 8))
 (segment (start 76.6126 79.9504) (end 75.6983 80.8647) (width 0.25) (layer "F.Cu") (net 8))
 (segment (start 70.6753 81.6726) (end 70.6753 82.04) (width 0.25) (layer "F.Cu") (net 8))
 (segment (start 102.7029 79.12) (end 79.0532 79.12) (width 0.25) (layer "F.Cu") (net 8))
 (segment (start 79.0532 79.12) (end 78.2228 79.9504) (width 0.25) (layer "F.Cu") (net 8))
 (segment (start 77.8146 79.5) (end 79.1299 78.1847) (width 0.25) (layer "F.Cu") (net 7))
 (segment (start 104.3625 71.1921) (end 104.3625 68.9466) (width 0.25) (layer "F.Cu") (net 7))
 (segment (start 97.3699 78.1847) (end 104.3625 71.1921) (width 0.25) (layer "F.Cu") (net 7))
 (segment (start 72.04 79.5) (end 77.8146 79.5) (width 0.25) (layer "F.Cu") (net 7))
 (segment (start 79.1299 78.1847) (end 97.3699 78.1847) (width 0.25) (layer "F.Cu") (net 7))
 (segment (start 77.1724 80.4008) (end 75.5332 82.04) (width 0.25) (layer "F.Cu") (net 9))
 (segment (start 80.397 79.9771) (end 79.3583 79.9771) (width 0.25) (layer "F.Cu") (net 9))
 (segment (start 79.3583 79.9771) (end 78.9346 80.4008) (width 0.25) (layer "F.Cu") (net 9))
 (segment (start 105.501 81.6156) (end 82.0355 81.6156) (width 0.25) (layer "F.Cu") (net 9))
 (segment (start 78.9346 80.4008) (end 77.1724 80.4008) (width 0.25) (layer "F.Cu") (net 9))
 (segment (start 75.5332 82.04) (end 72.04 82.04) (width 0.25) (layer "F.Cu") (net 9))
 (segment (start 82.0355 81.6156) (end 80.397 79.9771) (width 0.25) (layer "F.Cu") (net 9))
 (segment (start 69.5 87.12) (end 70.6753 87.12) (width 0.25) (layer "B.Cu") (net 12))
 (segment (start 70.6753 87.4874) (end 70.6753 87.12) (width 0.25) (layer "B.Cu") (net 12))
 (segment (start 73.9746 79.1281) (end 73.9746 86.8518) (width 0.25) (layer "B.Cu") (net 12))
 (segment (start 71.4832 88.2953) (end 70.6753 87.4874) (width 0.25) (layer "B.Cu") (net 12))
 (segment (start 72.5311 88.2953) (end 71.4832 88.2953) (width 0.25) (layer "B.Cu") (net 12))
 (segment (start 73.9746 86.8518) (end 72.5311 88.2953) (width 0.25) (layer "B.Cu") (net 12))
 (segment (start 79.2971 73.88) (end 79.2227 73.88) (width 0.25) (layer "B.Cu") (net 12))
 (segment (start 79.2227 73.88) (end 73.9746 79.1281) (width 0.25) (layer "B.Cu") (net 12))
 (segment (start 74.8054 83.4047) (end 71.4832 83.4047) (width 0.25) (layer "F.Cu") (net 10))
 (segment (start 77.0977 81.1124) (end 74.8054 83.4047) (width 0.25) (layer "F.Cu") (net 10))
 (segment (start 69.5 84.58) (end 70.6753 84.58) (width 0.25) (layer "F.Cu") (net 10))
 (segment (start 70.6753 84.2126) (end 70.6753 84.58) (width 0.25) (layer "F.Cu") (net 10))
 (segment (start 79.9299 81.1124) (end 77.0977 81.1124) (width 0.25) (layer "F.Cu") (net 10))
 (segment (start 71.4832 83.4047) (end 70.6753 84.2126) (width 0.25) (layer "F.Cu") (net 10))
 (segment (start 73.2153 85.1368) (end 72.4074 85.9447) (width 0.25) (layer "B.Cu") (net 13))
 (segment (start 73.2153 74.6681) (end 73.2153 85.1368) (width 0.25) (layer "B.Cu") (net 13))
 (segment (start 72.4074 85.9447) (end 72.04 85.9447) (width 0.25) (layer "B.Cu") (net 13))
 (segment (start 72.04 87.12) (end 72.04 85.9447) (width 0.25) (layer "B.Cu") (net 13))
 (segment (start 76.499 71.3844) (end 73.2153 74.6681) (width 0.25) (layer "B.Cu") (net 13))
 (segment (start 72.04 84.58) (end 73.2153 84.58) (width 0.25) (layer "F.Cu") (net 11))
 (segment (start 77.5072 83.9556) (end 73.8397 83.9556) (width 0.25) (layer "F.Cu") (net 11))
 (segment (start 73.8397 83.9556) (end 73.2153 84.58) (width 0.25) (layer "F.Cu") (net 11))
 (segment (start 77.6076 84.056) (end 77.5072 83.9556) (width 0.25) (layer "F.Cu") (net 11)))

